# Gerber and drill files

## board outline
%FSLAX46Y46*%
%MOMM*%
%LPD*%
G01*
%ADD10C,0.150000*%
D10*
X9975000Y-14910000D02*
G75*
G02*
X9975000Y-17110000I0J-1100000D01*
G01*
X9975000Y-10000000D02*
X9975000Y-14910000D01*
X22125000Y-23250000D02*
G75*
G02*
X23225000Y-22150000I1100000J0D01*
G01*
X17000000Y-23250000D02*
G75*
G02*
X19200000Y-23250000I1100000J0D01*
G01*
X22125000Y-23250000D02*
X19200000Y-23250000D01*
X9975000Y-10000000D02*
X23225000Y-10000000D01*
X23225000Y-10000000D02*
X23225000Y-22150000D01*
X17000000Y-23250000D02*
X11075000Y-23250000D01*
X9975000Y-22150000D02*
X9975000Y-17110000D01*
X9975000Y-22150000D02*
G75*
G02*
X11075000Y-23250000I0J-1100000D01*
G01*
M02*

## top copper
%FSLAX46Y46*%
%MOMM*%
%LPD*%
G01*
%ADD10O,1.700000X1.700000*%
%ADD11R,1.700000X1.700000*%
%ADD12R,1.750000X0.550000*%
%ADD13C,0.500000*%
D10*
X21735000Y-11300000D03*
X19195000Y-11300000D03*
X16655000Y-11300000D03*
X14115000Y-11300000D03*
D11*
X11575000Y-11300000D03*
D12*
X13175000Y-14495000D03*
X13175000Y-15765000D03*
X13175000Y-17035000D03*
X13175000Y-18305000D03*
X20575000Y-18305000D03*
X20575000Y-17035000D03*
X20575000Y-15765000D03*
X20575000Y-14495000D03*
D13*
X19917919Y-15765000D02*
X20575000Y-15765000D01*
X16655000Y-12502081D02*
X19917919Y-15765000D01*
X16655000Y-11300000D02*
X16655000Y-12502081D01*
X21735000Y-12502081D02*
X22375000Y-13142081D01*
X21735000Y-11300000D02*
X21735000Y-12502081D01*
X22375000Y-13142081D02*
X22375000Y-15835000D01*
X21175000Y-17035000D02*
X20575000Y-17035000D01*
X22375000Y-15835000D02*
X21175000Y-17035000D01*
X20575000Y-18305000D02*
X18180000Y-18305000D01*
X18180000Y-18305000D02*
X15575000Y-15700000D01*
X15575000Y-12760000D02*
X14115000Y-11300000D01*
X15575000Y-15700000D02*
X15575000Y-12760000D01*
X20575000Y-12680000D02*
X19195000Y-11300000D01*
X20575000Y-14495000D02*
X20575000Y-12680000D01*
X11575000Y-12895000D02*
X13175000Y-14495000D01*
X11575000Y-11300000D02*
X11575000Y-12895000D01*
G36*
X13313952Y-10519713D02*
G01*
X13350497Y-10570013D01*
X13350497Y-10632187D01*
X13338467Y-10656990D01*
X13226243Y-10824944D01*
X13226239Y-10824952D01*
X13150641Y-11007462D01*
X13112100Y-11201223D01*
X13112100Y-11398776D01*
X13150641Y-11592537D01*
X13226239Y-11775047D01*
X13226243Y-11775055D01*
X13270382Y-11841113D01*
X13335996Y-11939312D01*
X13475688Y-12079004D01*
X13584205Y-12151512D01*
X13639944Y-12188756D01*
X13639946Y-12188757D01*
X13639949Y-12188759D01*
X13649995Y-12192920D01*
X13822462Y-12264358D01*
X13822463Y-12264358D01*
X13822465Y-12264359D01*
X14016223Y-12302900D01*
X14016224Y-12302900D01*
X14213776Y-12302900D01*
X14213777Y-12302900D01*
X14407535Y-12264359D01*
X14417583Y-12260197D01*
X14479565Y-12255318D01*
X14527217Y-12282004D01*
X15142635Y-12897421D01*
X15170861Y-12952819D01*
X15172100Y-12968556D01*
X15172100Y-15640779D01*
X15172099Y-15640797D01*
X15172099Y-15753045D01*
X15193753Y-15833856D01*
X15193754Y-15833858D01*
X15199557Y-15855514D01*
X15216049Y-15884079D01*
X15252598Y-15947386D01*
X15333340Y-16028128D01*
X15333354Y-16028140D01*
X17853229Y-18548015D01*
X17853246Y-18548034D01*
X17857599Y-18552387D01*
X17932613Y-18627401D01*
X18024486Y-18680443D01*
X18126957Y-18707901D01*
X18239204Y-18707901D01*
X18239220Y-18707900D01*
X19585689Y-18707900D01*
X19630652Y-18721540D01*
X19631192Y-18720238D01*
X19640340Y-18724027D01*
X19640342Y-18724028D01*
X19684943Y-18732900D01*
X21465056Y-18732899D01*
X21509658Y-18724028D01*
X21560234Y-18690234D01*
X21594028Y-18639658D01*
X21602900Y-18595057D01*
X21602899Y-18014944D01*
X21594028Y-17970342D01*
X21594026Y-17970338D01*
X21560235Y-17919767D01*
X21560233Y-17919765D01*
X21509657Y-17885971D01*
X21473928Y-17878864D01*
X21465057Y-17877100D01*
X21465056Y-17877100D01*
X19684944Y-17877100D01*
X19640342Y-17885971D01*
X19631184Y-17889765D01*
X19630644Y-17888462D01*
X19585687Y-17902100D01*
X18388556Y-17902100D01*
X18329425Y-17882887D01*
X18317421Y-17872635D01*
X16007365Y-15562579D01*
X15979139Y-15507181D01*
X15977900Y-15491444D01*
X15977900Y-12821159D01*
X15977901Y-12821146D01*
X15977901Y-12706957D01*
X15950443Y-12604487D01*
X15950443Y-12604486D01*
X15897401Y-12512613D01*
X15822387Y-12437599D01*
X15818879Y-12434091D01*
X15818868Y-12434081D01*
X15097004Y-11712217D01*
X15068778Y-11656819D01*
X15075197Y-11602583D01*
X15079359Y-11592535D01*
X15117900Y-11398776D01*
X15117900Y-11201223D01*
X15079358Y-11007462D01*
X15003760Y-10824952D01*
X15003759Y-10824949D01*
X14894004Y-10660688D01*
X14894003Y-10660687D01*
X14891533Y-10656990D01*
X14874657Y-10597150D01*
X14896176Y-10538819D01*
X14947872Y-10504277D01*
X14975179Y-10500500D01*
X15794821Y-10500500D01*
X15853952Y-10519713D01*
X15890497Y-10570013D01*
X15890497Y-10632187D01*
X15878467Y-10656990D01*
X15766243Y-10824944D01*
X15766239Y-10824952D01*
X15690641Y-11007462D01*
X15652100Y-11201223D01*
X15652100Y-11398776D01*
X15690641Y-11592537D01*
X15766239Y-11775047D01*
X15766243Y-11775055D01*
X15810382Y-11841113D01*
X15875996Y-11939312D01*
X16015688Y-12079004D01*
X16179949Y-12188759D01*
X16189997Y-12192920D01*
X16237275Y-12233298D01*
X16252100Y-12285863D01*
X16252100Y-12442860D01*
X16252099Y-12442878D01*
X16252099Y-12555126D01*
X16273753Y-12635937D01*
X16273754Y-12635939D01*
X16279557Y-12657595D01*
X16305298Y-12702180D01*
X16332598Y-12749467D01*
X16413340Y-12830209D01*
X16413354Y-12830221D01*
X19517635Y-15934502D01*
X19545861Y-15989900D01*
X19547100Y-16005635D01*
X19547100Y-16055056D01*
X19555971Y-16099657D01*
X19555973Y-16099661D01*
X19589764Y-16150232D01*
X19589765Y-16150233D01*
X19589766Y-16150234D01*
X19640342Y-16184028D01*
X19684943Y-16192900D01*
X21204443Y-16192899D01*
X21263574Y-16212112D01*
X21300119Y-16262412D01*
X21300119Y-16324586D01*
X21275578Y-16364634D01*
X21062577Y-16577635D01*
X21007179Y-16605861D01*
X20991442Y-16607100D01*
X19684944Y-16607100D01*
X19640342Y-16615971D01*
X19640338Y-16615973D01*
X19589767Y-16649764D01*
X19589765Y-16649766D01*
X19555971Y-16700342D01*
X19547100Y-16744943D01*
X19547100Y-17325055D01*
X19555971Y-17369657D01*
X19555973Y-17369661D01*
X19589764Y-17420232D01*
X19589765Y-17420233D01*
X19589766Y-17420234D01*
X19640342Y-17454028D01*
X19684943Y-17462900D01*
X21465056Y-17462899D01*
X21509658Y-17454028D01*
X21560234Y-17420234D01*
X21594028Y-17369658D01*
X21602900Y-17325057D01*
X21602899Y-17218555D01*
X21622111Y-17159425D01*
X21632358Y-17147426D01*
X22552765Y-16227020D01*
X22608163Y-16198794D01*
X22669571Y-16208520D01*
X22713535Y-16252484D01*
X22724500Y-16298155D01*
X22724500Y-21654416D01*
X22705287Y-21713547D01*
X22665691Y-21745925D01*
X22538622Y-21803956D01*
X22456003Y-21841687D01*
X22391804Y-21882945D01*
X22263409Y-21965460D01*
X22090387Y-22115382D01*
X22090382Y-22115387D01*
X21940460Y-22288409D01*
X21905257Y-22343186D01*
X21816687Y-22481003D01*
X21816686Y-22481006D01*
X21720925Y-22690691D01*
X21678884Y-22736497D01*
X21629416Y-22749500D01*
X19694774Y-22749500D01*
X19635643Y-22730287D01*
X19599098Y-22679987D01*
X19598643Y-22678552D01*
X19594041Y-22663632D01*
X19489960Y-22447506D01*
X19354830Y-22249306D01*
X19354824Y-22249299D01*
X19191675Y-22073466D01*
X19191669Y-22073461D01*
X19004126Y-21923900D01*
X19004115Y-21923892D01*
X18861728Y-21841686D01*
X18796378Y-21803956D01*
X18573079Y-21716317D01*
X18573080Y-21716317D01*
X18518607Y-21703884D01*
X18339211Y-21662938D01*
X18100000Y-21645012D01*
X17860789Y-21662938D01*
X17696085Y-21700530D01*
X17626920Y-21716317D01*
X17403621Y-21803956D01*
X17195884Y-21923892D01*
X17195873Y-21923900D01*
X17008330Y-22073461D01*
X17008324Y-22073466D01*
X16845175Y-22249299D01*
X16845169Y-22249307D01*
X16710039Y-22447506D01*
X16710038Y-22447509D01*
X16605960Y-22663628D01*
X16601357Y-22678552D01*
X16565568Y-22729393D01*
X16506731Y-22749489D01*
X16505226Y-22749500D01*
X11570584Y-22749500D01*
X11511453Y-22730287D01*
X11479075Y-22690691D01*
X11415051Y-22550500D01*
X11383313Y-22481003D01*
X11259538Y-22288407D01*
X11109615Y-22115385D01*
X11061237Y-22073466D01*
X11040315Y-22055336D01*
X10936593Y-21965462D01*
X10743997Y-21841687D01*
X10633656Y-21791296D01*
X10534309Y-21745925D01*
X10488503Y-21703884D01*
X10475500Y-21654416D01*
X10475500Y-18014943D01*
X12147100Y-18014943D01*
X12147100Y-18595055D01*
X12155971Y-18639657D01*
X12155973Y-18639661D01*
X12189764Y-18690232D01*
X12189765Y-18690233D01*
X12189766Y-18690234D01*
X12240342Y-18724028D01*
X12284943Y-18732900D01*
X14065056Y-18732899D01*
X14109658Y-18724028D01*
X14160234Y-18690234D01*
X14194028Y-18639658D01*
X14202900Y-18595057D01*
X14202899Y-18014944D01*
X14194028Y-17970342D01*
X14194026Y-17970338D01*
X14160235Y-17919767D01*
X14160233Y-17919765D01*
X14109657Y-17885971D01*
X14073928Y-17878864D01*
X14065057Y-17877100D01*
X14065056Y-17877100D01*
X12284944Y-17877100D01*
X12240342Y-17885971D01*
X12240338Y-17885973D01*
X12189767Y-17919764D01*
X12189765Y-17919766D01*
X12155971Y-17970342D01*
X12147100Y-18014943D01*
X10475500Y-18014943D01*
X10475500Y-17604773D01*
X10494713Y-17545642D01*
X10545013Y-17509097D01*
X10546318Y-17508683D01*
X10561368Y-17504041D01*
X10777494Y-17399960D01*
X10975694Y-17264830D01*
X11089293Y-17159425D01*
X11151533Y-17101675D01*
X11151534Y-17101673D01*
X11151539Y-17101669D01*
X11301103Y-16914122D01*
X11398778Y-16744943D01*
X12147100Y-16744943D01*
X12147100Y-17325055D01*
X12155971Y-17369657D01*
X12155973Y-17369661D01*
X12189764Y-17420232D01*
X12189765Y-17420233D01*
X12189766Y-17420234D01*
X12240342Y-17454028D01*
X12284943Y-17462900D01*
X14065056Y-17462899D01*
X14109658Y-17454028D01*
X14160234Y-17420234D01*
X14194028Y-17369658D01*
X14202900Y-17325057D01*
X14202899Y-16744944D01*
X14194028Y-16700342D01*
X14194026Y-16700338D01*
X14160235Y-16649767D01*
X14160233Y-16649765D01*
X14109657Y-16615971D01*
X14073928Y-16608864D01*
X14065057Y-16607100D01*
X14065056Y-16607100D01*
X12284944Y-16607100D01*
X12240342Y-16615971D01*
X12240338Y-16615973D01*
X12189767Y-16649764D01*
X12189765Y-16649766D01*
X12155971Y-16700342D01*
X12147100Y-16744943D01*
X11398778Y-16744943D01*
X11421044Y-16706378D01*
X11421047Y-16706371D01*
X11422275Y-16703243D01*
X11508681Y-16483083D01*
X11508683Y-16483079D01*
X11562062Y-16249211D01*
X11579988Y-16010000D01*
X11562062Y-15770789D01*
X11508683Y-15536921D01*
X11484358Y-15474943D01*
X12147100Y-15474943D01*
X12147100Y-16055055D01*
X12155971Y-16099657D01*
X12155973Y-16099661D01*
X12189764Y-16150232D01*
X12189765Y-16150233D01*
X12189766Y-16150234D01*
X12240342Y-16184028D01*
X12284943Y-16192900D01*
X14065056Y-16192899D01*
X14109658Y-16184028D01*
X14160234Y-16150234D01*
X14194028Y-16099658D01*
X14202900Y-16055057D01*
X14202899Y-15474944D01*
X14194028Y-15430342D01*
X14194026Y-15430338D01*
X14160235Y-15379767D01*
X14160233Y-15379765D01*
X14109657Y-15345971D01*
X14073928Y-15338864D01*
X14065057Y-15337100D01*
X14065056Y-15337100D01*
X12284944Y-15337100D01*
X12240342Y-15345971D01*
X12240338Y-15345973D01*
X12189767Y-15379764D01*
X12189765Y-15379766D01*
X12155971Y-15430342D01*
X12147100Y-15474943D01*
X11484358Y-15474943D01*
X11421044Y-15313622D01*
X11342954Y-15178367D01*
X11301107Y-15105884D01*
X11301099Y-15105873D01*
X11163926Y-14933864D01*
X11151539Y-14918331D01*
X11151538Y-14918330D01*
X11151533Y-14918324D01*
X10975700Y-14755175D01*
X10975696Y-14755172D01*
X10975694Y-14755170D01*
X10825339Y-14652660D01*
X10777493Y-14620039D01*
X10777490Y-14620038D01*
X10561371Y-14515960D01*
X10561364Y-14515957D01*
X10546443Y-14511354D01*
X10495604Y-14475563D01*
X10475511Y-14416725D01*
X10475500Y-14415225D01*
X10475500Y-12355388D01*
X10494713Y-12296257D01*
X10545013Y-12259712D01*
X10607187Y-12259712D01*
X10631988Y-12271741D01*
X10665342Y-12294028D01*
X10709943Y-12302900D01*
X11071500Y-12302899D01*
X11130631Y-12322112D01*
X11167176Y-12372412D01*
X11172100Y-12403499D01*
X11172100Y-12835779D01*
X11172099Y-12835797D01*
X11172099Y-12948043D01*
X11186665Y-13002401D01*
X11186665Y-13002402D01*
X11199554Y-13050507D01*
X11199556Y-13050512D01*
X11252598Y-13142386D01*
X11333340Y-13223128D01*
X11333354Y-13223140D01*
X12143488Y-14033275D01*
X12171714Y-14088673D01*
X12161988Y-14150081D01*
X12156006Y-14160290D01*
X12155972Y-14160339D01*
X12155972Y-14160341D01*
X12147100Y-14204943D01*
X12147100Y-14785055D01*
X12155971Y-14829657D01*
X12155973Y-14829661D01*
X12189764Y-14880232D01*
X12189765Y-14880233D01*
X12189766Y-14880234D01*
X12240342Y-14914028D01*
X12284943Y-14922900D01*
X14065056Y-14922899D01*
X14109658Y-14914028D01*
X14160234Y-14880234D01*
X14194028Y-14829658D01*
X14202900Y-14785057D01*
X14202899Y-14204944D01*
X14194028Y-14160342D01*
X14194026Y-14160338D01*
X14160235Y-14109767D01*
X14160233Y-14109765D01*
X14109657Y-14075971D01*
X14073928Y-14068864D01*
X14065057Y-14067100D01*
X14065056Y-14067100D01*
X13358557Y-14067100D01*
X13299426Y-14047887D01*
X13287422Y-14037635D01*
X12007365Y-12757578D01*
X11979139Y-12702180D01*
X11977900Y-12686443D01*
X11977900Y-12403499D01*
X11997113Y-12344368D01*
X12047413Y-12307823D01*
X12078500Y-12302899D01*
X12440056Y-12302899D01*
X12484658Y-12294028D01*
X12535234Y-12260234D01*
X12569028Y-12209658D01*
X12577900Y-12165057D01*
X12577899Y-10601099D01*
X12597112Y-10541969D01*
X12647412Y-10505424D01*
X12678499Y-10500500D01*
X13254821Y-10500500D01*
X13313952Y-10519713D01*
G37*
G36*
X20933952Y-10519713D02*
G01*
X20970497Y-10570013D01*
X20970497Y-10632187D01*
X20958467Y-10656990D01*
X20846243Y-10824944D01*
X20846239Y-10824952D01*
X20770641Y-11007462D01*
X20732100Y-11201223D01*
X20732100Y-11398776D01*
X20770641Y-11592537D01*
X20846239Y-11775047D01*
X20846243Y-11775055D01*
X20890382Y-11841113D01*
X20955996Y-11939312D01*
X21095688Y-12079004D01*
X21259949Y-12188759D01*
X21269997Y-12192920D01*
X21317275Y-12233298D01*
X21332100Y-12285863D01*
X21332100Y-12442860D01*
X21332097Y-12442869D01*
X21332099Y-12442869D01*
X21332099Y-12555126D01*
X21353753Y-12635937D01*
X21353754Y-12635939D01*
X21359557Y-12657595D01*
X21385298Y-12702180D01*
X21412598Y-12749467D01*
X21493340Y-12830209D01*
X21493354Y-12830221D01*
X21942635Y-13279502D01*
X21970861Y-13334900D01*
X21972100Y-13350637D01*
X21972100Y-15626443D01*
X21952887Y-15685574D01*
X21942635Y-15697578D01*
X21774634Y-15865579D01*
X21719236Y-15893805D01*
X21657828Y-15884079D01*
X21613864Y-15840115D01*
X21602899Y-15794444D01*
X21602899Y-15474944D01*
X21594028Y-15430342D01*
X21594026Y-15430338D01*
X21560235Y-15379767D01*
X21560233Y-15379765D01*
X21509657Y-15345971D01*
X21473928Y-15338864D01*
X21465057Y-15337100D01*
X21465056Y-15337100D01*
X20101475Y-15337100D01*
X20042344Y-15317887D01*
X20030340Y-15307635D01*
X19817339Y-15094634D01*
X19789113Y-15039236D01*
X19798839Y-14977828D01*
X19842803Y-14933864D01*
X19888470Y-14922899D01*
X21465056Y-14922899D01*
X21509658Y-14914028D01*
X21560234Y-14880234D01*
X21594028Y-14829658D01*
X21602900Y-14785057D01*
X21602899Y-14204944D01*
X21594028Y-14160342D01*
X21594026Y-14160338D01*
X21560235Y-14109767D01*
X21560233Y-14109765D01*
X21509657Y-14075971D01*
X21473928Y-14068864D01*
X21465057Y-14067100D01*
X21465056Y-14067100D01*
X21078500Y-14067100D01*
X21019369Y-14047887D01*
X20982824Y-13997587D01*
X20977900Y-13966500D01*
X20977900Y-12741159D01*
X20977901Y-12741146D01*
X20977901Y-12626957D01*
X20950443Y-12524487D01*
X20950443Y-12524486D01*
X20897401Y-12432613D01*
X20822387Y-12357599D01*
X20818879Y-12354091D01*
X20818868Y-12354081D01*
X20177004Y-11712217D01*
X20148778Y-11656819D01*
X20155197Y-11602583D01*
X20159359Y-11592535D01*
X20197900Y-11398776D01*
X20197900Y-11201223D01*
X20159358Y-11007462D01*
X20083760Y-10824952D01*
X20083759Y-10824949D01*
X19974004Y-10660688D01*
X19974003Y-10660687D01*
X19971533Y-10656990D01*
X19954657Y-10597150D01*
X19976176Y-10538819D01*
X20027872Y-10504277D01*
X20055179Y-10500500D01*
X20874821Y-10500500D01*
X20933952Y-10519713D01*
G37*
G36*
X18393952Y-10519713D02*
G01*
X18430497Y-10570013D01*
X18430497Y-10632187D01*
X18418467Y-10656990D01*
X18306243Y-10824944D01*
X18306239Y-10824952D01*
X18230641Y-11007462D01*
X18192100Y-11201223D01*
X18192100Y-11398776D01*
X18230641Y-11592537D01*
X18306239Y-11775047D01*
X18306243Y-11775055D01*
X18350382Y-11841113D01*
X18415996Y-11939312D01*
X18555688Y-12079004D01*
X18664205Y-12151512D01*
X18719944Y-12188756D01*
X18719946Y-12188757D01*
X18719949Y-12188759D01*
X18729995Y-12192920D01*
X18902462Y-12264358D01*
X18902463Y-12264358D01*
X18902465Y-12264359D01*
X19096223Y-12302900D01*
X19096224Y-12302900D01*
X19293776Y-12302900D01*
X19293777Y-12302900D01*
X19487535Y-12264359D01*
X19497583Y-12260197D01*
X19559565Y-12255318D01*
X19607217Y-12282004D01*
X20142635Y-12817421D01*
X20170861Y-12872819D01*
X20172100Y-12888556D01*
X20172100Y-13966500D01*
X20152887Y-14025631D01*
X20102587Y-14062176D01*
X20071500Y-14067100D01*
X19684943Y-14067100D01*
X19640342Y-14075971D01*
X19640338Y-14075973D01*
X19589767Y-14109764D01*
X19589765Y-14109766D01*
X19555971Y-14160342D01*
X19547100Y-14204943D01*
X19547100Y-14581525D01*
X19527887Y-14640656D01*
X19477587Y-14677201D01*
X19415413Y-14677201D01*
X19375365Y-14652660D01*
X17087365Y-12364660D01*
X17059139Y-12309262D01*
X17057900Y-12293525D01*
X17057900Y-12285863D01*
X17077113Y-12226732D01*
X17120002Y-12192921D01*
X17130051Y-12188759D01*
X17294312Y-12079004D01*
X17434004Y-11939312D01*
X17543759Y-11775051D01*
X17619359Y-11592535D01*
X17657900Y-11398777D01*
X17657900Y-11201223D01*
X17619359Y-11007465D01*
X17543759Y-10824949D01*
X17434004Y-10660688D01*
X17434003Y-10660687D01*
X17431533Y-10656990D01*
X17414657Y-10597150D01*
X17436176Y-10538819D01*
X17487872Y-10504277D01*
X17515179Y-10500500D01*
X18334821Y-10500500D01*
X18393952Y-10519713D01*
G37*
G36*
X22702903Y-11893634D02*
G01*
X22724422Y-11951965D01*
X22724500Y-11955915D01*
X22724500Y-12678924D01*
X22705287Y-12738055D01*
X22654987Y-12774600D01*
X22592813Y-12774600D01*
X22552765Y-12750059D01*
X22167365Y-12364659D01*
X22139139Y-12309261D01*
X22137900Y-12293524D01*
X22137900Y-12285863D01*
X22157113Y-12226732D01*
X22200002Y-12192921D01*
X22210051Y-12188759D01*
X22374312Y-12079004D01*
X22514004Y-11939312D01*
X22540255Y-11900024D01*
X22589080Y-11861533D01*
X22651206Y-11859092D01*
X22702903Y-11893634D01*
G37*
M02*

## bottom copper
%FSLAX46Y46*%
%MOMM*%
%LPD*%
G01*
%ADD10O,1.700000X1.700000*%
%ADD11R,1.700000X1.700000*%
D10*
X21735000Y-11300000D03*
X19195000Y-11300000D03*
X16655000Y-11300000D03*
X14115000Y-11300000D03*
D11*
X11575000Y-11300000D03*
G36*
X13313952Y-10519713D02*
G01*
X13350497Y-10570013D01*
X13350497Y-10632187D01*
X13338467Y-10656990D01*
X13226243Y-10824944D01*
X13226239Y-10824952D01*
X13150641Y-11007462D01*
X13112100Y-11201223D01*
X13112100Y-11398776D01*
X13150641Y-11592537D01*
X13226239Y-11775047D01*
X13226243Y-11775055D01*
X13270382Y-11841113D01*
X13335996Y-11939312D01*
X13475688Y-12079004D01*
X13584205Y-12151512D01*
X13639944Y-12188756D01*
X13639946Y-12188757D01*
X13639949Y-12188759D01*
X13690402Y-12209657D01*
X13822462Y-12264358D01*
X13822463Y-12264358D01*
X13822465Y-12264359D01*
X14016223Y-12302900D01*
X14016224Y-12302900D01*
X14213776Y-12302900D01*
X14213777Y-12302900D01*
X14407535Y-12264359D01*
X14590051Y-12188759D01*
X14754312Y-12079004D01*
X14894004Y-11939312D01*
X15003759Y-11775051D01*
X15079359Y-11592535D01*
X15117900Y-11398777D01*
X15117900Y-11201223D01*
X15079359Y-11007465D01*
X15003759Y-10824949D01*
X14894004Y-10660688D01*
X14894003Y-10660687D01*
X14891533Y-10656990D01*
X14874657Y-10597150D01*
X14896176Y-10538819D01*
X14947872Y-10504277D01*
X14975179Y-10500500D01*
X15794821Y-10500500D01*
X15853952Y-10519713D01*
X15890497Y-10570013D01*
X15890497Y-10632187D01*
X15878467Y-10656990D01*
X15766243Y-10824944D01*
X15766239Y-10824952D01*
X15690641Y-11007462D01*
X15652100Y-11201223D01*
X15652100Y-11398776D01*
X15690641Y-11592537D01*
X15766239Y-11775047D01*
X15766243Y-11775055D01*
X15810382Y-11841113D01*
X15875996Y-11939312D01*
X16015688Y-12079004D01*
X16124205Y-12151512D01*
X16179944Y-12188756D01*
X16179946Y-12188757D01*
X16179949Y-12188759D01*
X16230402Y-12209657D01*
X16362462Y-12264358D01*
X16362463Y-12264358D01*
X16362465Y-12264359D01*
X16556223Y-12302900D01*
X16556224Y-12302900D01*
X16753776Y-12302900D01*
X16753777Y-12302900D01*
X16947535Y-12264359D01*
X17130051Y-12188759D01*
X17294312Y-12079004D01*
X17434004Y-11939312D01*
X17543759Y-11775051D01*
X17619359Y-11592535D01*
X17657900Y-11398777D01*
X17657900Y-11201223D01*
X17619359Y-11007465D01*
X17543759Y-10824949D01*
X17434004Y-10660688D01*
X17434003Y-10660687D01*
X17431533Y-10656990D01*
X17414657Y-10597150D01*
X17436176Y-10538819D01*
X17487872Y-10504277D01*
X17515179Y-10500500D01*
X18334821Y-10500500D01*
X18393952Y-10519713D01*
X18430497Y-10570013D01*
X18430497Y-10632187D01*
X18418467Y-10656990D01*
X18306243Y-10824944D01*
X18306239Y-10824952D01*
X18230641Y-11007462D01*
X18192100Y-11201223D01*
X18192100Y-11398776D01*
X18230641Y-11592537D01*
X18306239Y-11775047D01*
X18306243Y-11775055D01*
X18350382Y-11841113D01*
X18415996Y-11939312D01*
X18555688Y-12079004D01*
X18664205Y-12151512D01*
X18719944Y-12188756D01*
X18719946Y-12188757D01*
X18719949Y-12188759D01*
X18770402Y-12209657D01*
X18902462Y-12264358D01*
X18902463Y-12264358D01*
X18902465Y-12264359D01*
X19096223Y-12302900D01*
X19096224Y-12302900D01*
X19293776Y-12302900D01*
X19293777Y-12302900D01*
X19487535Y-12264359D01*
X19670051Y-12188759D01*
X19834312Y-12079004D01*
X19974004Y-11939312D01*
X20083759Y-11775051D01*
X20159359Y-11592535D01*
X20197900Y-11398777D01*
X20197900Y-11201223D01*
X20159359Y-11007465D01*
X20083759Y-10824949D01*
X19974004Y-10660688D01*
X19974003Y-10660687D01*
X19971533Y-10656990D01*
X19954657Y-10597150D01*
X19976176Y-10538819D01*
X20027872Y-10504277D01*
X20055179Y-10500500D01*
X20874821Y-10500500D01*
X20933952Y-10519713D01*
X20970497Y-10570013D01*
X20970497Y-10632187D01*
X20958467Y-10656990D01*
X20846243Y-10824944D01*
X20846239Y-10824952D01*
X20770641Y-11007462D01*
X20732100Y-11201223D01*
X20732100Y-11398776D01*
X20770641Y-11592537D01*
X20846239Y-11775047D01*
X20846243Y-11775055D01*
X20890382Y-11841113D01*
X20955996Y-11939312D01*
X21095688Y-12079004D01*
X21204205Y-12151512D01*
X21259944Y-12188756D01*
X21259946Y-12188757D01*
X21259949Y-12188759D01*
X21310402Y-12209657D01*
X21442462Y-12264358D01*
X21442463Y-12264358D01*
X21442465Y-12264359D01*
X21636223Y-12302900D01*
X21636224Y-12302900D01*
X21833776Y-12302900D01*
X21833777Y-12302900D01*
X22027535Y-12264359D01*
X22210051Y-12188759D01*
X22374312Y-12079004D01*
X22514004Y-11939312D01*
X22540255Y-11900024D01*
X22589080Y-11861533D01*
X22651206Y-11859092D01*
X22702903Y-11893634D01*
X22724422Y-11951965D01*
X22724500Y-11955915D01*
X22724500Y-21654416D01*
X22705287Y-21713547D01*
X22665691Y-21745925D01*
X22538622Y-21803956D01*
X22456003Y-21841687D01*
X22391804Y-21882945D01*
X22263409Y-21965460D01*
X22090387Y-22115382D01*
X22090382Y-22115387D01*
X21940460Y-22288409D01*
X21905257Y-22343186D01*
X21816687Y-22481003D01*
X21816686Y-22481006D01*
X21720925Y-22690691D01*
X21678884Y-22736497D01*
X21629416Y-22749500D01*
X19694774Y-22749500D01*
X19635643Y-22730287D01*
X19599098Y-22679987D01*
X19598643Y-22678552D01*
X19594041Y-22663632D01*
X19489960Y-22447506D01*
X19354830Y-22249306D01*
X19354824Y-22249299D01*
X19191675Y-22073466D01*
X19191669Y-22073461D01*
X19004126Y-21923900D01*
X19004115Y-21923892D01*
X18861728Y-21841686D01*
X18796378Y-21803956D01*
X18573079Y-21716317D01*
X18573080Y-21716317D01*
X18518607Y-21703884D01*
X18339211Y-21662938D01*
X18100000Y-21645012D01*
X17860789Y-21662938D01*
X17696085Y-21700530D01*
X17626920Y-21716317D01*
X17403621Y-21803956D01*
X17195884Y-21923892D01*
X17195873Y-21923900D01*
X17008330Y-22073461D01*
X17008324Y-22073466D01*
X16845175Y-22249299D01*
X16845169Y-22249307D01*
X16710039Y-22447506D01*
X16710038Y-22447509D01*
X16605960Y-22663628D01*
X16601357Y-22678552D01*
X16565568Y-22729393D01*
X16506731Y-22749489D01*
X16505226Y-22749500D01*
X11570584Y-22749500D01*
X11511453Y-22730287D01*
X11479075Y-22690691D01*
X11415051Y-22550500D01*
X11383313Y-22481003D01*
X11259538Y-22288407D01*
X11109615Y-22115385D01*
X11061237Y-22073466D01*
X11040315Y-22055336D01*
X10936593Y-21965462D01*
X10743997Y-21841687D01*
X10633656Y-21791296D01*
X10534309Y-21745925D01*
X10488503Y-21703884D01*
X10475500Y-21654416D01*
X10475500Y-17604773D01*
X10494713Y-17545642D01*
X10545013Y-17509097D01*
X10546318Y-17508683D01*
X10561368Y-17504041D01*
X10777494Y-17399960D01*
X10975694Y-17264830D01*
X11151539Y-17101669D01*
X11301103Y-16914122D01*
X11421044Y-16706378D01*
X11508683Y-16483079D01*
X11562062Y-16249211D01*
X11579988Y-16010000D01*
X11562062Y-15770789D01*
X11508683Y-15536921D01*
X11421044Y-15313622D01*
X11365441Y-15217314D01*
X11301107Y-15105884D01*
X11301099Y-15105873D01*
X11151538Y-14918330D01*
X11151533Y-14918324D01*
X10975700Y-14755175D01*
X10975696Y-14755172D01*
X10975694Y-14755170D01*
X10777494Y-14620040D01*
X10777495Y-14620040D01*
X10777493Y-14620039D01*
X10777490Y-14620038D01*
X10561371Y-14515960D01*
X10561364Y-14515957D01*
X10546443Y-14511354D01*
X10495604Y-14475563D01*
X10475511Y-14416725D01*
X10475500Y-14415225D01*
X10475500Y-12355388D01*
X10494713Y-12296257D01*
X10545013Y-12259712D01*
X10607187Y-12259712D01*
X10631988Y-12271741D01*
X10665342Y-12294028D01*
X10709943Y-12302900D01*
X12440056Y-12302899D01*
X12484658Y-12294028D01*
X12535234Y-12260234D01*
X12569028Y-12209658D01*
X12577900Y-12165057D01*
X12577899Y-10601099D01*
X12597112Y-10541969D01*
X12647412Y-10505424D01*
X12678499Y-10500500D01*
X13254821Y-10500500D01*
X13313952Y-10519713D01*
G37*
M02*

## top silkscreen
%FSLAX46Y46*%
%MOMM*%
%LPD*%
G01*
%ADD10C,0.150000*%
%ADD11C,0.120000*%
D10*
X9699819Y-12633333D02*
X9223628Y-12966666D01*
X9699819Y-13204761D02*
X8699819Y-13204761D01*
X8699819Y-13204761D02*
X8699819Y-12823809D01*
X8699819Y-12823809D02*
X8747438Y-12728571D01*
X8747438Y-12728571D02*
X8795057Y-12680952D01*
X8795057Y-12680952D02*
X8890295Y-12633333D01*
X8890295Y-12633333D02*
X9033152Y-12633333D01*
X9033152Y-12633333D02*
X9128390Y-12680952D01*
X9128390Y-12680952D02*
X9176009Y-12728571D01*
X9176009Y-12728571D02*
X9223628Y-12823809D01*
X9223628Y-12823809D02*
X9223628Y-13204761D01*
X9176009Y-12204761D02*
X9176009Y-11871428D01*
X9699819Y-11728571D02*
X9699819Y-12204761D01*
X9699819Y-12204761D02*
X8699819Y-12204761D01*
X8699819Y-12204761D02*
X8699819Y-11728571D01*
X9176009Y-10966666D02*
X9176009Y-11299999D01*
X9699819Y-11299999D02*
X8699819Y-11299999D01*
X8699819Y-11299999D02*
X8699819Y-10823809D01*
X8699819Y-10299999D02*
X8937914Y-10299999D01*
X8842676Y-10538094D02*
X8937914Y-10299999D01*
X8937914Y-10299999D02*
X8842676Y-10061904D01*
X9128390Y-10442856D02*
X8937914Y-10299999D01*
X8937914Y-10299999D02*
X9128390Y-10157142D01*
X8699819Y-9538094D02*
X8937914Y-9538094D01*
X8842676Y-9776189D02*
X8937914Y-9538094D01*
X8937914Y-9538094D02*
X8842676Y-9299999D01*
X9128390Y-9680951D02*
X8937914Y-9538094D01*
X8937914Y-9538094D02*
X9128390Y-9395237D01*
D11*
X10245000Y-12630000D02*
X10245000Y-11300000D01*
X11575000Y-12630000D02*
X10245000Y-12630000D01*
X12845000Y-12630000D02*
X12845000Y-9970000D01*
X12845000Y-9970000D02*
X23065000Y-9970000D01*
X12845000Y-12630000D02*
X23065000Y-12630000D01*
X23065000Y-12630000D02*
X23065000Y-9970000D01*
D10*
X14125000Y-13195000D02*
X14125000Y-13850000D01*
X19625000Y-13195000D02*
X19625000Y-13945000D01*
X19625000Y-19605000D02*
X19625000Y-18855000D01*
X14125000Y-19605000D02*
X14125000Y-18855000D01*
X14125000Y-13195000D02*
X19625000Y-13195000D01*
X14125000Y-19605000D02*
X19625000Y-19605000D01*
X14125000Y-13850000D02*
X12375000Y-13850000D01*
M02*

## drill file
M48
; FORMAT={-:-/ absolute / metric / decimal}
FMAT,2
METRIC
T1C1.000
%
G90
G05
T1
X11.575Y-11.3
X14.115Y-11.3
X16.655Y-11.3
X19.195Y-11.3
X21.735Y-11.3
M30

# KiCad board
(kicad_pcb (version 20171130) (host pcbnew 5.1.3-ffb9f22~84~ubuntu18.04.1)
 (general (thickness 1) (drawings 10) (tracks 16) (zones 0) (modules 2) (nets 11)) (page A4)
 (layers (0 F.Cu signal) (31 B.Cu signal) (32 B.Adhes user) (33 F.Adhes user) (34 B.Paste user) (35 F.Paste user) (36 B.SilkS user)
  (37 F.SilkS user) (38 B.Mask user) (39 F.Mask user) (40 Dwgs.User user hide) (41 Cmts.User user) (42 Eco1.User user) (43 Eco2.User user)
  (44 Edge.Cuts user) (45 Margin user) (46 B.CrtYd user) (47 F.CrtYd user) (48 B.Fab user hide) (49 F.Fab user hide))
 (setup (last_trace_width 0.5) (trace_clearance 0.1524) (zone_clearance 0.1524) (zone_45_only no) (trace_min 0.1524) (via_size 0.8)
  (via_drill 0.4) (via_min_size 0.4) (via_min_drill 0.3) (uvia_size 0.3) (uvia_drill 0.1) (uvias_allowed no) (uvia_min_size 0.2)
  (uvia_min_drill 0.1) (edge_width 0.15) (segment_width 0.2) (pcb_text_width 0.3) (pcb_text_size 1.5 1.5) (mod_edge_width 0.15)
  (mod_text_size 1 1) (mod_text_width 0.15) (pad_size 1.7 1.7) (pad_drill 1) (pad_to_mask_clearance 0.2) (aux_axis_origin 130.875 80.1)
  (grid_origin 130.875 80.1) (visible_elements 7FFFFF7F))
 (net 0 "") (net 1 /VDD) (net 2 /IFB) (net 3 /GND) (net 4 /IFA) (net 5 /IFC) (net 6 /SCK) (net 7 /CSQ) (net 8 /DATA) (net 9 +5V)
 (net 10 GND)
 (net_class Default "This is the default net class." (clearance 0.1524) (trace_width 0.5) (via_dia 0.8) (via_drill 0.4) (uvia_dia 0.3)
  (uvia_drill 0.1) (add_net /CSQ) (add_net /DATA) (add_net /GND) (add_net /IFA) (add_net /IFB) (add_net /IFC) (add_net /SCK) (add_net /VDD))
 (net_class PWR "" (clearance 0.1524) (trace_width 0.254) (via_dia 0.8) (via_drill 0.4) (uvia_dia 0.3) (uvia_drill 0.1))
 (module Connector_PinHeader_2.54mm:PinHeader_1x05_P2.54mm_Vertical (layer F.Cu) (at 11.575 11.3 90)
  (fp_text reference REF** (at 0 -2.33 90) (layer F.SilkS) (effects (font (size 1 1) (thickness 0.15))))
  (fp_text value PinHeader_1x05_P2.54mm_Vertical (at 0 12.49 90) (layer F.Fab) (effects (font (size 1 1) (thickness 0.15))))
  (fp_line (start -1.33 -1.33) (end 0 -1.33) (layer F.SilkS) (width 0.12))
  (fp_line (start -1.33 0) (end -1.33 -1.33) (layer F.SilkS) (width 0.12))
  (fp_line (start -1.33 1.27) (end 1.33 1.27) (layer F.SilkS) (width 0.12))
  (fp_line (start 1.33 1.27) (end 1.33 11.49) (layer F.SilkS) (width 0.12))
  (fp_line (start -1.33 1.27) (end -1.33 11.49) (layer F.SilkS) (width 0.12))
  (fp_line (start -1.33 11.49) (end 1.33 11.49) (layer F.SilkS) (width 0.12))
  (pad 5 thru_hole oval (at 0 10.16 90) (size 1.7 1.7) (drill 1) (layers *.Cu *.Mask) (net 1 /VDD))
  (pad 4 thru_hole oval (at 0 7.62 90) (size 1.7 1.7) (drill 1) (layers *.Cu *.Mask) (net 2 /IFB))
  (pad 3 thru_hole oval (at 0 5.08 90) (size 1.7 1.7) (drill 1) (layers *.Cu *.Mask) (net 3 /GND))
  (pad 2 thru_hole oval (at 0 2.54 90) (size 1.7 1.7) (drill 1) (layers *.Cu *.Mask) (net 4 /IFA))
  (pad 1 thru_hole rect (at 0 0 90) (size 1.7 1.7) (drill 1) (layers *.Cu *.Mask) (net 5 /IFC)))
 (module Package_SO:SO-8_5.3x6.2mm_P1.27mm (layer F.Cu) (at 16.875 16.4)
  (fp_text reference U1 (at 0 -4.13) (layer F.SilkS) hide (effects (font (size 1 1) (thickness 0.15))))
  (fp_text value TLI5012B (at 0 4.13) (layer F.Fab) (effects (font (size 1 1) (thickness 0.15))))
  (fp_line (start -2.75 -3.205) (end -2.75 -2.55) (layer F.SilkS) (width 0.15))
  (fp_line (start 2.75 -3.205) (end 2.75 -2.455) (layer F.SilkS) (width 0.15))
  (fp_line (start 2.75 3.205) (end 2.75 2.455) (layer F.SilkS) (width 0.15))
  (fp_line (start -2.75 3.205) (end -2.75 2.455) (layer F.SilkS) (width 0.15))
  (fp_line (start -2.75 -3.205) (end 2.75 -3.205) (layer F.SilkS) (width 0.15))
  (fp_line (start -2.75 3.205) (end 2.75 3.205) (layer F.SilkS) (width 0.15))
  (fp_line (start -2.75 -2.55) (end -4.5 -2.55) (layer F.SilkS) (width 0.15))
  (pad 1 smd rect (at -3.7 -1.905) (size 1.75 0.55) (layers F.Cu F.Paste F.Mask) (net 5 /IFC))
  (pad 2 smd rect (at -3.7 -0.635) (size 1.75 0.55) (layers F.Cu F.Paste F.Mask) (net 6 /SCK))
  (pad 3 smd rect (at -3.7 0.635) (size 1.75 0.55) (layers F.Cu F.Paste F.Mask) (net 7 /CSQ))
  (pad 4 smd rect (at -3.7 1.905) (size 1.75 0.55) (layers F.Cu F.Paste F.Mask) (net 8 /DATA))
  (pad 5 smd rect (at 3.7 1.905) (size 1.75 0.55) (layers F.Cu F.Paste F.Mask) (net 4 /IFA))
  (pad 6 smd rect (at 3.7 0.635) (size 1.75 0.55) (layers F.Cu F.Paste F.Mask) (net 1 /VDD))
  (pad 7 smd rect (at 3.7 -0.635) (size 1.75 0.55) (layers F.Cu F.Paste F.Mask) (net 3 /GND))
  (pad 8 smd rect (at 3.7 -1.905) (size 1.75 0.55) (layers F.Cu F.Paste F.Mask) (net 2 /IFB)))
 (gr_arc (start 9.975 16.01) (end 9.975 14.91) (angle 180) (layer Edge.Cuts) (width 0.15))
 (gr_line (start 9.975 10) (end 9.975 14.91) (angle 90) (layer Edge.Cuts) (width 0.15))
 (gr_arc (start 23.225 23.25) (end 22.125 23.25) (angle 90) (layer Edge.Cuts) (width 0.15))
 (gr_arc (start 18.1 23.25) (end 17 23.25) (angle 180) (layer Edge.Cuts) (width 0.15))
 (gr_line (start 22.125 23.25) (end 19.2 23.25) (angle 90) (layer Edge.Cuts) (width 0.15))
 (gr_line (start 9.975 10) (end 23.225 10) (angle 90) (layer Edge.Cuts) (width 0.15))
 (gr_line (start 23.225 10) (end 23.225 22.15) (angle 90) (layer Edge.Cuts) (width 0.15))
 (gr_line (start 17 23.25) (end 11.075 23.25) (angle 90) (layer Edge.Cuts) (width 0.15))
 (gr_line (start 9.975 22.15) (end 9.975 17.11) (angle 90) (layer Edge.Cuts) (width 0.15))
 (gr_arc (start 9.975 23.25) (end 9.975 22.15) (angle 90) (layer Edge.Cuts) (width 0.15))
 (segment (start 19.917919 15.765) (end 20.575 15.765) (width 0.5) (layer F.Cu) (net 3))
 (segment (start 16.655 12.502081) (end 19.917919 15.765) (width 0.5) (layer F.Cu) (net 3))
 (segment (start 16.655 11.3) (end 16.655 12.502081) (width 0.5) (layer F.Cu) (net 3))
 (segment (start 21.735 12.502081) (end 22.375 13.142081) (width 0.5) (layer F.Cu) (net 1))
 (segment (start 21.735 11.3) (end 21.735 12.502081) (width 0.5) (layer F.Cu) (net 1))
 (segment (start 22.375 13.142081) (end 22.375 15.835) (width 0.5) (layer F.Cu) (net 1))
 (segment (start 21.175 17.035) (end 20.575 17.035) (width 0.5) (layer F.Cu) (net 1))
 (segment (start 22.375 15.835) (end 21.175 17.035) (width 0.5) (layer F.Cu) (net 1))
 (segment (start 20.575 18.305) (end 18.18 18.305) (width 0.5) (layer F.Cu) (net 4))
 (segment (start 18.18 18.305) (end 15.575 15.7) (width 0.5) (layer F.Cu) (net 4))
 (segment (start 15.575 12.76) (end 14.115 11.3) (width 0.5) (layer F.Cu) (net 4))
 (segment (start 15.575 15.7) (end 15.575 12.76) (width 0.5) (layer F.Cu) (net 4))
 (segment (start 20.575 12.68) (end 19.195 11.3) (width 0.5) (layer F.Cu) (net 2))
 (segment (start 20.575 14.495) (end 20.575 12.68) (width 0.5) (layer F.Cu) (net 2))
 (segment (start 11.575 12.895) (end 13.175 14.495) (width 0.5) (layer F.Cu) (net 5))
 (segment (start 11.575 11.3) (end 11.575 12.895) (width 0.5) (layer F.Cu) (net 5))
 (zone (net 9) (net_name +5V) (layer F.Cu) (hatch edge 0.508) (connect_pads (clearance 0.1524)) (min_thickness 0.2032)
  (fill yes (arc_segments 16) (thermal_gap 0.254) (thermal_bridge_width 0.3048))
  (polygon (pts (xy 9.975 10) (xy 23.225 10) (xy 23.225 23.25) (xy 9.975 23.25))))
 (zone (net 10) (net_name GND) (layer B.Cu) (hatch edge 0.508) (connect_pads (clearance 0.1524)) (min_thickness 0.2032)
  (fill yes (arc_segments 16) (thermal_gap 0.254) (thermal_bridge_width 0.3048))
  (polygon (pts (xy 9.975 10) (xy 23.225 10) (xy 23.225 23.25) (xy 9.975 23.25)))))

